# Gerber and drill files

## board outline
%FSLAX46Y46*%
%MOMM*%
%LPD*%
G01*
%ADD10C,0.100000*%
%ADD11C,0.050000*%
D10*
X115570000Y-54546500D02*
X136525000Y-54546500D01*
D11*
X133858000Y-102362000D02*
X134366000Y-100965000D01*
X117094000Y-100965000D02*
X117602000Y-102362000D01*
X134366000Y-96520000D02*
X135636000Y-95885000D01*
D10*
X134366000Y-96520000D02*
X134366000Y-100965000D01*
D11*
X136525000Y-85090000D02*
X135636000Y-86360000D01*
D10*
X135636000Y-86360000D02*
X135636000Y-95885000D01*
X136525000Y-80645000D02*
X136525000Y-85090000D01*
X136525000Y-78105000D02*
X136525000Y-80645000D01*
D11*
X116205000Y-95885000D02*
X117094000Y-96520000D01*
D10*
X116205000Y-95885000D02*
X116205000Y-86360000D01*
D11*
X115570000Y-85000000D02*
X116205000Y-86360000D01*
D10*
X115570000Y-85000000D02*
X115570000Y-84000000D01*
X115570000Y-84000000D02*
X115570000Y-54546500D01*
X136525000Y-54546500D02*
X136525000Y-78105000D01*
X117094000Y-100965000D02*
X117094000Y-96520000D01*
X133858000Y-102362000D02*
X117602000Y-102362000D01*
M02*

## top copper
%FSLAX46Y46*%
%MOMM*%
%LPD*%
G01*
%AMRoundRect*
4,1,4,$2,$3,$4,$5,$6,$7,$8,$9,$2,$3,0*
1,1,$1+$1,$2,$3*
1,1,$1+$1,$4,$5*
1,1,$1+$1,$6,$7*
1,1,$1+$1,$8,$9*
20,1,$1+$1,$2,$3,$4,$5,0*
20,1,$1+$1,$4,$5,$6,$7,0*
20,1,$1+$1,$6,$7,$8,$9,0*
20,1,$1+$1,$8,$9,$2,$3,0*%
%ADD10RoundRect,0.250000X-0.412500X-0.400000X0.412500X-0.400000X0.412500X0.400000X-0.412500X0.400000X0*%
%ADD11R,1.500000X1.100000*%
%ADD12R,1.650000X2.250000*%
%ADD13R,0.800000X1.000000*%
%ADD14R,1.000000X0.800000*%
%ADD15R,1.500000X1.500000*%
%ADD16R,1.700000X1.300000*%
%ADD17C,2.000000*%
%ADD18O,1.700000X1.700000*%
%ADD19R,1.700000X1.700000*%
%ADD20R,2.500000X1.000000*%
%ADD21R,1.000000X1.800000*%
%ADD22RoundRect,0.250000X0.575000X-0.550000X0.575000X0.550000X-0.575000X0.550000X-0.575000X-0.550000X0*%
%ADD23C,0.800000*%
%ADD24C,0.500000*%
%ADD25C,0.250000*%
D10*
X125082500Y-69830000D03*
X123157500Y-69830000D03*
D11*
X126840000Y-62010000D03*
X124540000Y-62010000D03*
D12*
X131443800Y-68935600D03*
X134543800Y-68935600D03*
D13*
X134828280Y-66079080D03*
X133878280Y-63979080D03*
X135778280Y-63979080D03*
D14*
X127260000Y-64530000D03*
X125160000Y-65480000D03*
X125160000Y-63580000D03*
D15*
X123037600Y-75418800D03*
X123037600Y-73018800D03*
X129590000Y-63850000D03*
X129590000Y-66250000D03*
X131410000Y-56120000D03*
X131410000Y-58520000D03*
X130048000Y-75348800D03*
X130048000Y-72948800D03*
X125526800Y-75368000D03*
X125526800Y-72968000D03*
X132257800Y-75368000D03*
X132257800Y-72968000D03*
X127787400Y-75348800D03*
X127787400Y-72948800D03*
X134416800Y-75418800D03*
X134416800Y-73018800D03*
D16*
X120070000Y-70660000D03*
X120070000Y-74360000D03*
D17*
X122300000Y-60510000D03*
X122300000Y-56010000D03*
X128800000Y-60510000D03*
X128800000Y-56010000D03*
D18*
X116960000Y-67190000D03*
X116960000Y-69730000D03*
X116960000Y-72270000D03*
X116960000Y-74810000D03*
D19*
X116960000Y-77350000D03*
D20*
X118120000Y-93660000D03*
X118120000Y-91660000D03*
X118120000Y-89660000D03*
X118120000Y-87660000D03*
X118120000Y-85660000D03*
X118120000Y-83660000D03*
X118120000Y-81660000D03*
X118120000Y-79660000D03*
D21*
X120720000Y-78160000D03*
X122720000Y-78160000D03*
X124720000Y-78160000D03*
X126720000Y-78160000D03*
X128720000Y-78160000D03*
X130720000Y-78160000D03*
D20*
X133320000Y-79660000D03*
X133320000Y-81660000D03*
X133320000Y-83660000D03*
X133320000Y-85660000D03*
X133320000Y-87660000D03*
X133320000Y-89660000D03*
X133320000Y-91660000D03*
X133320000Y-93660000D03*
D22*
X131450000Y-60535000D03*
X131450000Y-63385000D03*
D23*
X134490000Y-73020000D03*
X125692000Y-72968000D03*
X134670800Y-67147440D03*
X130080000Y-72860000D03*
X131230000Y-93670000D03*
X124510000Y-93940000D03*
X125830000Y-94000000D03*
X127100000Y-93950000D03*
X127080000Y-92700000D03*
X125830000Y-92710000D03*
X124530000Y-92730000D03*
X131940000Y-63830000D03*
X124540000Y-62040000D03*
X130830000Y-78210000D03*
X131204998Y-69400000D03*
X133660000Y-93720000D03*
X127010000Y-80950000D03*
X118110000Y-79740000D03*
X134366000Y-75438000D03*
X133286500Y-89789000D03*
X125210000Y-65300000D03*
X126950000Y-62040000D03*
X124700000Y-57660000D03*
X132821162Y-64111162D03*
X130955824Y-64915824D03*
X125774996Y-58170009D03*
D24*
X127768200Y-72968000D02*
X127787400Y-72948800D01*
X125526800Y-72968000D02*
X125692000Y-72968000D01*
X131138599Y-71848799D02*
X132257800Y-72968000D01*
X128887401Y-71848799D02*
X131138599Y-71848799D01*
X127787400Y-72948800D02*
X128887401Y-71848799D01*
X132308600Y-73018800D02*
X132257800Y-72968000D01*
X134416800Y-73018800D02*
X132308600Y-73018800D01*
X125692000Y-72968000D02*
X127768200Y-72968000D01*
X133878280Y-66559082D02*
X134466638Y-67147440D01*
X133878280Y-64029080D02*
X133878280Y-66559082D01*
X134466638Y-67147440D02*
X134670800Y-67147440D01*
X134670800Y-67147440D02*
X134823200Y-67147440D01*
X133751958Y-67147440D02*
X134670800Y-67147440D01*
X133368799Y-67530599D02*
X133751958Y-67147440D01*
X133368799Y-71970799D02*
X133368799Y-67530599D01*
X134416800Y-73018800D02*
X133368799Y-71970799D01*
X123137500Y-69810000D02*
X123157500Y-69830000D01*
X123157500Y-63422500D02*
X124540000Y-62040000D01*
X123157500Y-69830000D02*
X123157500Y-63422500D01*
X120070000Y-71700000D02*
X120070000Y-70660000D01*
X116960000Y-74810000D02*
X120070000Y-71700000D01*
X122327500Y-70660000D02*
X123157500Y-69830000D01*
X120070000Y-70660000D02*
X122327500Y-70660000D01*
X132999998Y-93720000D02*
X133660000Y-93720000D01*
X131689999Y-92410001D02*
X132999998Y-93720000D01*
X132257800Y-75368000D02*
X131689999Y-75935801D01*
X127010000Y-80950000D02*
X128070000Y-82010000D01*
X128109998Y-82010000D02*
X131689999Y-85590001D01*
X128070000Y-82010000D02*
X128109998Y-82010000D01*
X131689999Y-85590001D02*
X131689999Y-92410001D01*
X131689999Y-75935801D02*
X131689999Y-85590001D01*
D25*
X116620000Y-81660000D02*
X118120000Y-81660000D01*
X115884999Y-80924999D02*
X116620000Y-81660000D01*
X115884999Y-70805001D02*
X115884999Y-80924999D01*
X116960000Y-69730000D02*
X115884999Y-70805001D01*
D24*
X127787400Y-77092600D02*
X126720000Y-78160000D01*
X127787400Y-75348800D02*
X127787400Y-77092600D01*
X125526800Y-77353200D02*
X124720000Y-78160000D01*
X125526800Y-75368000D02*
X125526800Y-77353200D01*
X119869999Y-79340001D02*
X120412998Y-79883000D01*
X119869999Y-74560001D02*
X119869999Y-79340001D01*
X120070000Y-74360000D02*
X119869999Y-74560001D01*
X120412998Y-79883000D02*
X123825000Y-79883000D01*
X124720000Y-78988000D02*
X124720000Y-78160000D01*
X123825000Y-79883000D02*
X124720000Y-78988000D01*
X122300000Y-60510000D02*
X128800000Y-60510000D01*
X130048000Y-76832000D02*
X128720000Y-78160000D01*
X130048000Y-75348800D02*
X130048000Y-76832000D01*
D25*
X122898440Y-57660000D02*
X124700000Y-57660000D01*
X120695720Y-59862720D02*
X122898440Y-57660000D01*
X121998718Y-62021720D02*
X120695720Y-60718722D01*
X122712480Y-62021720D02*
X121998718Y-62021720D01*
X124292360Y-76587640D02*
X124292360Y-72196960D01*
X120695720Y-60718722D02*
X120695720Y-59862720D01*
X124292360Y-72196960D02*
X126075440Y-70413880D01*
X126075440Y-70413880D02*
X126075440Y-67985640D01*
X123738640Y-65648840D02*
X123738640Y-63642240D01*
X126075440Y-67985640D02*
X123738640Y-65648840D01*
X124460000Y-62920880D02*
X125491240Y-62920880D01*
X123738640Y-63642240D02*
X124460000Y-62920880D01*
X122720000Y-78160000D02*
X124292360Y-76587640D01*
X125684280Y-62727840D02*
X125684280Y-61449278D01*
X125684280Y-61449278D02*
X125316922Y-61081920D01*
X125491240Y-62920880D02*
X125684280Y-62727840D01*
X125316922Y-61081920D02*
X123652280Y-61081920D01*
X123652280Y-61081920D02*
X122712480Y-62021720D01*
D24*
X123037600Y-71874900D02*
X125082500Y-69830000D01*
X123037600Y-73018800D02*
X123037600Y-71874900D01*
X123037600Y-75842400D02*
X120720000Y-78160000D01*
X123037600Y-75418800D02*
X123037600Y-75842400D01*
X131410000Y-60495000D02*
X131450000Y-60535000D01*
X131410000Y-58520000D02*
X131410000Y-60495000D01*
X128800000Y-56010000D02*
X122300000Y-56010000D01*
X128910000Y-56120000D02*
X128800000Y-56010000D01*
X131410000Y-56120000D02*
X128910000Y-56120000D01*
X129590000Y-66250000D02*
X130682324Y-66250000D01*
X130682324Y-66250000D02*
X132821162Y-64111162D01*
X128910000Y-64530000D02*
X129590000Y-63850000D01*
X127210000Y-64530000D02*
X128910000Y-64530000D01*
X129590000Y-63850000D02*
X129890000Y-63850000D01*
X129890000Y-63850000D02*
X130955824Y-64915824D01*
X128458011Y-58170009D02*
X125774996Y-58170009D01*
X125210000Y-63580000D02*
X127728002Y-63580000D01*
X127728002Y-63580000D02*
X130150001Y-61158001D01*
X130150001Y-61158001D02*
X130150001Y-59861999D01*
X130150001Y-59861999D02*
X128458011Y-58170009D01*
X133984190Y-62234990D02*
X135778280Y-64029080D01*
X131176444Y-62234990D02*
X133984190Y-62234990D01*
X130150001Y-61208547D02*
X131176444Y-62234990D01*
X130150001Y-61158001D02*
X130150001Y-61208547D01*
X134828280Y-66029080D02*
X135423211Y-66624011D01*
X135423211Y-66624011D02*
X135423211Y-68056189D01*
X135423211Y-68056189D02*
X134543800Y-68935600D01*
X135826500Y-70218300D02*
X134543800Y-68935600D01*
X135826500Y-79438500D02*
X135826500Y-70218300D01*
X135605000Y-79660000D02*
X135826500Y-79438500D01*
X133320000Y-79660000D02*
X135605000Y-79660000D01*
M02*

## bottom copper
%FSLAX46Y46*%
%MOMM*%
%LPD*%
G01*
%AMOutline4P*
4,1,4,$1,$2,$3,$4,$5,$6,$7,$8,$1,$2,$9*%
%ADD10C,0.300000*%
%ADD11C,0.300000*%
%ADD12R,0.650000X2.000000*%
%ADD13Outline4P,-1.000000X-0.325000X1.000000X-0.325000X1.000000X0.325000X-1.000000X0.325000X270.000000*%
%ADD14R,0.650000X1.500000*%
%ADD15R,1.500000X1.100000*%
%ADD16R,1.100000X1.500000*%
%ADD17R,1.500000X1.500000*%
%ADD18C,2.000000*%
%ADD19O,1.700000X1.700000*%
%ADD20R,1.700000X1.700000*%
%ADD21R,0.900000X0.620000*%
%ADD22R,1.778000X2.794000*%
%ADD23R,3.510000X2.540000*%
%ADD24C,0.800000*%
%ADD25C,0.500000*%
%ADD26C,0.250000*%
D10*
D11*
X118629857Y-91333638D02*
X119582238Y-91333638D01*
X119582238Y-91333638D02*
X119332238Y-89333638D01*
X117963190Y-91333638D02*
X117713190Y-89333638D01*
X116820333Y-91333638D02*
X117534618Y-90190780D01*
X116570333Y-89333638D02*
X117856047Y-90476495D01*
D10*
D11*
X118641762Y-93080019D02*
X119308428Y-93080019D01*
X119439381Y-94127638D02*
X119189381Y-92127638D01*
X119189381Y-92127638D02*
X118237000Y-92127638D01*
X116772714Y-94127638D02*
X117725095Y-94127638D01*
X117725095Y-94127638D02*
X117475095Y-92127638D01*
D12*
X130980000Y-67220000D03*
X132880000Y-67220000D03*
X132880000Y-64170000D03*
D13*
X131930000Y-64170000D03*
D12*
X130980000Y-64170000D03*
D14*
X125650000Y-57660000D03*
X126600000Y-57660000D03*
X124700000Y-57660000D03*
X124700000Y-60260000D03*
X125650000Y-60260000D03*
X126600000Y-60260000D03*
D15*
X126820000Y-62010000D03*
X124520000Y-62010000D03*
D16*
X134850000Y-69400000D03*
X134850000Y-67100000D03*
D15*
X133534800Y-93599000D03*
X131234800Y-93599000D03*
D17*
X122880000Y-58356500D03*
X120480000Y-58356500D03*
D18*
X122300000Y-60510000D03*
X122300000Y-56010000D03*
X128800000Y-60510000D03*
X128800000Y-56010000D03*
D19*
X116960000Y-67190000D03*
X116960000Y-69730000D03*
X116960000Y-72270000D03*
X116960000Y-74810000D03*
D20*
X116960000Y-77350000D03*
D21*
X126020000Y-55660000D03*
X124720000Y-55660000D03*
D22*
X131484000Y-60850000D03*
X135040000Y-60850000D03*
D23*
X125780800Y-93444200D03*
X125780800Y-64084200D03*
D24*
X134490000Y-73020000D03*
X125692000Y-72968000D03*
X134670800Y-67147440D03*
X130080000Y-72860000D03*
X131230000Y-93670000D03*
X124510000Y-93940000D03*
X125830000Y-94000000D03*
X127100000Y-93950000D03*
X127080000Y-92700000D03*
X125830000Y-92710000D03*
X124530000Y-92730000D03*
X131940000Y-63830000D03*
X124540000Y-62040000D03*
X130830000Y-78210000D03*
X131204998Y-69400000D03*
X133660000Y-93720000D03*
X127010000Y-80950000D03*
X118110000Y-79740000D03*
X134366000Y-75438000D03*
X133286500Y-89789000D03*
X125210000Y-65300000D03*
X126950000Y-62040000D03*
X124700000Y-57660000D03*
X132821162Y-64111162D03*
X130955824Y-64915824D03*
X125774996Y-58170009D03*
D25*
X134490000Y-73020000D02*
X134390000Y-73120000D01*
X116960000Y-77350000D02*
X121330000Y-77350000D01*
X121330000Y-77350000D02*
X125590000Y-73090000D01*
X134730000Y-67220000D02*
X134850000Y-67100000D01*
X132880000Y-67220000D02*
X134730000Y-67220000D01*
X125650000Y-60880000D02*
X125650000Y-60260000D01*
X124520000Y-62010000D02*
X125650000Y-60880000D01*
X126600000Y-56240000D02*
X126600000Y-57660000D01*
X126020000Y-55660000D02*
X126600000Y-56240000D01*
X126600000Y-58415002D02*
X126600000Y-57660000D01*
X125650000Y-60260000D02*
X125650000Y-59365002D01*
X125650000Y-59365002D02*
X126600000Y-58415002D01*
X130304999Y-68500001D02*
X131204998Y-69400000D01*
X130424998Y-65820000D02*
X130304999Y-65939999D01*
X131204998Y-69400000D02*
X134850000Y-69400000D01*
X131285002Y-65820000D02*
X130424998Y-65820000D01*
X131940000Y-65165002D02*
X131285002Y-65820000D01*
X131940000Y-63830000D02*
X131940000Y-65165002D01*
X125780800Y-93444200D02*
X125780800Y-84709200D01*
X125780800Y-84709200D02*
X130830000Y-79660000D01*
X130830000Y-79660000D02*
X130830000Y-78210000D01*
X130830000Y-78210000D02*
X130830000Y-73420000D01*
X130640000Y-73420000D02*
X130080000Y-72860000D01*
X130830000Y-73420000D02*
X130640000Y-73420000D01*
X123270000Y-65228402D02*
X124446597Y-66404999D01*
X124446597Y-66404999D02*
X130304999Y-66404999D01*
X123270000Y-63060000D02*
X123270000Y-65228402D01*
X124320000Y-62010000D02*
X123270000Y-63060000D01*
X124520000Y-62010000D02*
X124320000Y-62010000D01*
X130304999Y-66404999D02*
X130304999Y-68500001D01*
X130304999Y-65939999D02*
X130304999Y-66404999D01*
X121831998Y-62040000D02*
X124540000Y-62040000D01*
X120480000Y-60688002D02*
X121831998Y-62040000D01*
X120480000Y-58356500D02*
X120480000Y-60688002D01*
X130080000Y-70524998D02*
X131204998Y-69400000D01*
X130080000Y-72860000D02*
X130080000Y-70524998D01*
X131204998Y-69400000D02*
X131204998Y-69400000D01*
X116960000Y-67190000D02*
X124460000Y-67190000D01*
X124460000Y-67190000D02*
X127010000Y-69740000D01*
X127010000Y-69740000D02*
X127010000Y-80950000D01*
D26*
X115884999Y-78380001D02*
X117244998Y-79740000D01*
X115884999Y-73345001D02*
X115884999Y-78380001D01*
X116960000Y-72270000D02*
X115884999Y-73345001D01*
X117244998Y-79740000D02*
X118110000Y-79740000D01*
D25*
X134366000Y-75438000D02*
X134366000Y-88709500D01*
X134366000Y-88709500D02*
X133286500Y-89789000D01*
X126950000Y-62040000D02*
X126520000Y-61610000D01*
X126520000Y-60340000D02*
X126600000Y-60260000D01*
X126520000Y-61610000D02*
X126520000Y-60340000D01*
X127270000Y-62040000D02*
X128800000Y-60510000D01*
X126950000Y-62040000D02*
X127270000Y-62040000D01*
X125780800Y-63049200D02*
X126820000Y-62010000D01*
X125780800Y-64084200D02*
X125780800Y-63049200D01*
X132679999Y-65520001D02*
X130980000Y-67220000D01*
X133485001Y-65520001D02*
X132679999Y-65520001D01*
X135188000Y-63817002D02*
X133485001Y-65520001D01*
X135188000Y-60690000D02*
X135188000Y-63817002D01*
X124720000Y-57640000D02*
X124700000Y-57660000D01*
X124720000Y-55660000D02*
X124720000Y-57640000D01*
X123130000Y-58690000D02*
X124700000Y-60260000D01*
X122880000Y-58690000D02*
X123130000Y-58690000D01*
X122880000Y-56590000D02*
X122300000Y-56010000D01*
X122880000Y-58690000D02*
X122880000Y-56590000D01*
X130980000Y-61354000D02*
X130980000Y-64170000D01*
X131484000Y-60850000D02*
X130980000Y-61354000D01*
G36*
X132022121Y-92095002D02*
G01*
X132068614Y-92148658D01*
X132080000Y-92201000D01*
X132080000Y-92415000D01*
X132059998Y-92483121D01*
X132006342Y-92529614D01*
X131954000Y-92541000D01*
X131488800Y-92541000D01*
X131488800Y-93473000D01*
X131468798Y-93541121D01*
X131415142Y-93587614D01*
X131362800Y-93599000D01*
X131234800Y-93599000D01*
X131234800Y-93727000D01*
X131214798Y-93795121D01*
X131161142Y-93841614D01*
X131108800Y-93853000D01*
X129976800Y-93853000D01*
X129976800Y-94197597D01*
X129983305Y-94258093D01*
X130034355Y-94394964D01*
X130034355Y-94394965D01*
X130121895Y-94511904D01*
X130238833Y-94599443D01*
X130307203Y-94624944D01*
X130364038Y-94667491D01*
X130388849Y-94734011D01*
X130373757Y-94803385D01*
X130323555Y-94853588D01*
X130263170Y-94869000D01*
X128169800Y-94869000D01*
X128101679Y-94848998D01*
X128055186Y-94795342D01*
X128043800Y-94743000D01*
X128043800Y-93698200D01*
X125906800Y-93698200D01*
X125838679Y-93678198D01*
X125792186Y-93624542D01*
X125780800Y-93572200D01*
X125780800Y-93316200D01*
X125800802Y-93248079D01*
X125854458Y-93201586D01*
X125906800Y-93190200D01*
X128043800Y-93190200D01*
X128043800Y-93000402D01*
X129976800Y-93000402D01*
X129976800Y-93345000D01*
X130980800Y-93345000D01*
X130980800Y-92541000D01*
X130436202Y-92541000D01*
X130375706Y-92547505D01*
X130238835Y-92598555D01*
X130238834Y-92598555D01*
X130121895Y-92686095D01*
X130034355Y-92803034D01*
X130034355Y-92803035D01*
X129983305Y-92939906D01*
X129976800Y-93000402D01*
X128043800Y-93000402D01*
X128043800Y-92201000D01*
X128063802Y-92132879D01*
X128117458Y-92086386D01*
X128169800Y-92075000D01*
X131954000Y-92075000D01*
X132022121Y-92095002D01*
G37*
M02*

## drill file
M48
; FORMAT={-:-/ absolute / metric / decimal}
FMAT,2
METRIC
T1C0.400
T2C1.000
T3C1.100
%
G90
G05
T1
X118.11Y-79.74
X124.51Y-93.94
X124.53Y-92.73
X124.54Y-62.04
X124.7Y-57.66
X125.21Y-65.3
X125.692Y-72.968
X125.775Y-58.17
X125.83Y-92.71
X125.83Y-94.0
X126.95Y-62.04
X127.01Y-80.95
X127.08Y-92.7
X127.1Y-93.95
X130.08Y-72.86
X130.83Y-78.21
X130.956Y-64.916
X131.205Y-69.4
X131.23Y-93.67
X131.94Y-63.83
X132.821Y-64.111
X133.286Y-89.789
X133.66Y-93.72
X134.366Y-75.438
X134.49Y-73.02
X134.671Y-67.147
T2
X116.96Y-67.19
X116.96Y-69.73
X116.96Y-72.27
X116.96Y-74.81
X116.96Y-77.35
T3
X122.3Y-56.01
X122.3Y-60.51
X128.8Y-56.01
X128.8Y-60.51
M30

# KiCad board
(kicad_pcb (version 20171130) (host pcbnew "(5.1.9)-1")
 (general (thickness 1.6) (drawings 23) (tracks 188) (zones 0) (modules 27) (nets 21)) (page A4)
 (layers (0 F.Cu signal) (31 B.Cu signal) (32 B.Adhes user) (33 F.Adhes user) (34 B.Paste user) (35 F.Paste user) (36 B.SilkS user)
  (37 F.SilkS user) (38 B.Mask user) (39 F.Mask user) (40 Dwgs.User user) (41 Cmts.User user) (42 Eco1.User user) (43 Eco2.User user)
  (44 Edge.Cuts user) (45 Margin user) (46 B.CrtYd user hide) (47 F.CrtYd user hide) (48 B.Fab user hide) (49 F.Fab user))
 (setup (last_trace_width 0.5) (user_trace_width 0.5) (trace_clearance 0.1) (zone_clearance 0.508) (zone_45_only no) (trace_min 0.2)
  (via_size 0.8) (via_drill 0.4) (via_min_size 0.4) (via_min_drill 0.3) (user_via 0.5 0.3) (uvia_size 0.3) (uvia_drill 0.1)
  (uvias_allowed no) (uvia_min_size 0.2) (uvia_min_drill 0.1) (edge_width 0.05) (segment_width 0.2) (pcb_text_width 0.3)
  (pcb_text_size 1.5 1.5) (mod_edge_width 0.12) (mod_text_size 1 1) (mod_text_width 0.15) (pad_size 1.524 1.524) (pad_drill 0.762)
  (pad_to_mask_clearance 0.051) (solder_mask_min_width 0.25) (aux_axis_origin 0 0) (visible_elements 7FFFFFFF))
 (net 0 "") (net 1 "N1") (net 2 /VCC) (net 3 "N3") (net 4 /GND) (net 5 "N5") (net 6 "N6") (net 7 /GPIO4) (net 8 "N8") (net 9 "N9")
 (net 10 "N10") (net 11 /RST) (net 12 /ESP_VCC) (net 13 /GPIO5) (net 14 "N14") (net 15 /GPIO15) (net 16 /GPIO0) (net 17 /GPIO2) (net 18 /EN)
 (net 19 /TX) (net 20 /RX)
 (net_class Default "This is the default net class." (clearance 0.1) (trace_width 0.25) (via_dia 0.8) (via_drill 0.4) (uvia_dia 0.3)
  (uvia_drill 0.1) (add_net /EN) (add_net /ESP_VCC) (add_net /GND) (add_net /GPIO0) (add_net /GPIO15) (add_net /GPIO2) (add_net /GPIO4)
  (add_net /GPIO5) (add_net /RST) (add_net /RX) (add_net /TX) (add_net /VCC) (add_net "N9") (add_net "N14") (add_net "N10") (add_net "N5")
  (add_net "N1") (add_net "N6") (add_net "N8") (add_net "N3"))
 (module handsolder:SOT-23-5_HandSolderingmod (layer B.Cu) (at 131.93 65.72 270)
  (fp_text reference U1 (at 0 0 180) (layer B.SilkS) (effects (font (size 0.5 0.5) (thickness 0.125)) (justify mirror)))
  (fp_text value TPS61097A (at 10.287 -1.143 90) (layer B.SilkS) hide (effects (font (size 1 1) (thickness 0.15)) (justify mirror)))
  (pad 5 smd rect (at 1.5 0.95 270) (size 2 0.65) (layers B.Cu B.Paste B.Mask) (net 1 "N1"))
  (pad 4 smd rect (at 1.5 -0.95 270) (size 2 0.65) (layers B.Cu B.Paste B.Mask) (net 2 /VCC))
  (pad 3 smd rect (at -1.55 -0.95 270) (size 2 0.65) (layers B.Cu B.Paste B.Mask) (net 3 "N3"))
  (pad 2 smd trapezoid (at -1.55 0 270) (size 2 0.65) (layers B.Cu B.Paste B.Mask) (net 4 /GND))
  (pad 1 smd rect (at -1.55 0.95 270) (size 2 0.65) (layers B.Cu B.Paste B.Mask) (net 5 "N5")))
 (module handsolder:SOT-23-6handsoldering (layer B.Cu) (at 125.65 58.96 90)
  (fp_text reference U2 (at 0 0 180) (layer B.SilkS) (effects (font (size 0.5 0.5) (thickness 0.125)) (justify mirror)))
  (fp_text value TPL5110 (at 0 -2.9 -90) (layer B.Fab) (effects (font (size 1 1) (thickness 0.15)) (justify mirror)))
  (pad 5 smd rect (at 1.3 0 90) (size 1.5 0.65) (layers B.Cu B.Paste B.Mask) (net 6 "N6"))
  (pad 6 smd rect (at 1.3 0.95 90) (size 1.5 0.65) (layers B.Cu B.Paste B.Mask) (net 4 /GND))
  (pad 4 smd rect (at 1.3 -0.95 90) (size 1.5 0.65) (layers B.Cu B.Paste B.Mask) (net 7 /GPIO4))
  (pad 3 smd rect (at -1.3 -0.95 90) (size 1.5 0.65) (layers B.Cu B.Paste B.Mask) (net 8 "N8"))
  (pad 2 smd rect (at -1.3 0 90) (size 1.5 0.65) (layers B.Cu B.Paste B.Mask) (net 4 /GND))
  (pad 1 smd rect (at -1.3 0.95 90) (size 1.5 0.65) (layers B.Cu B.Paste B.Mask) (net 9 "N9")))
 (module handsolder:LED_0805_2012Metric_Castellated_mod (layer F.Cu) (at 124.12 69.83)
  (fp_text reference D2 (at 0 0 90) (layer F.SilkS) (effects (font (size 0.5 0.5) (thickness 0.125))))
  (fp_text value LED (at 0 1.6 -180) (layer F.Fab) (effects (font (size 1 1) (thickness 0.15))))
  (pad 2 smd roundrect (at 0.9625 0) (size 1.325 1.3) (layers F.Cu F.Paste F.Mask) (roundrect_rratio 0.1923076923076923) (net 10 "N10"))
  (pad 1 smd roundrect (at -0.9625 0) (size 1.325 1.3) (layers F.Cu F.Paste F.Mask) (roundrect_rratio 0.1923076923076923) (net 4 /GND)))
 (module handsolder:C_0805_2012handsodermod (layer F.Cu) (at 125.69 62.01)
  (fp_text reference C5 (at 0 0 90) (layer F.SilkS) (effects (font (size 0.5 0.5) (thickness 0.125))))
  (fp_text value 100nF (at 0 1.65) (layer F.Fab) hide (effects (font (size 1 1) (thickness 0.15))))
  (pad 2 smd rect (at 1.15 0) (size 1.5 1.1) (layers F.Cu F.Paste F.Mask) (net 9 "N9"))
  (pad 1 smd rect (at -1.15 0) (size 1.5 1.1) (layers F.Cu F.Paste F.Mask) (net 4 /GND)))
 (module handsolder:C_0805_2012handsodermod (layer B.Cu) (at 125.67 62.01)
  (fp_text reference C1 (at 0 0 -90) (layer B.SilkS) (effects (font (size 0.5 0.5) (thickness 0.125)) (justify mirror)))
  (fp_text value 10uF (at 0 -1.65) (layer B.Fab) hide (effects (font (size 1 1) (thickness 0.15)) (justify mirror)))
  (pad 2 smd rect (at 1.15 0) (size 1.5 1.1) (layers B.Cu B.Paste B.Mask) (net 9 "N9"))
  (pad 1 smd rect (at -1.15 0) (size 1.5 1.1) (layers B.Cu B.Paste B.Mask) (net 4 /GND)))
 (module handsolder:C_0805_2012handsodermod (layer B.Cu) (at 134.85 68.25 270)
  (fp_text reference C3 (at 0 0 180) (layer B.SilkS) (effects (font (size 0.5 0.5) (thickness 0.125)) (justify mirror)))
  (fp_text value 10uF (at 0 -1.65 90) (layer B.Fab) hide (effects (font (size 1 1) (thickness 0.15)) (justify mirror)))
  (pad 2 smd rect (at 1.15 0 270) (size 1.5 1.1) (layers B.Cu B.Paste B.Mask) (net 4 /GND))
  (pad 1 smd rect (at -1.15 0 270) (size 1.5 1.1) (layers B.Cu B.Paste B.Mask) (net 2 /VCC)))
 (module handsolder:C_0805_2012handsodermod (layer B.Cu) (at 132.3848 93.599)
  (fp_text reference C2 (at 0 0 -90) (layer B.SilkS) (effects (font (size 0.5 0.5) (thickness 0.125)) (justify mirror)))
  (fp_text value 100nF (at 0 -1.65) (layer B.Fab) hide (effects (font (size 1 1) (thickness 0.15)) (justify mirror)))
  (pad 2 smd rect (at 1.15 0) (size 1.5 1.1) (layers B.Cu B.Paste B.Mask) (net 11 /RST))
  (pad 1 smd rect (at -1.15 0) (size 1.5 1.1) (layers B.Cu B.Paste B.Mask) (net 4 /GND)))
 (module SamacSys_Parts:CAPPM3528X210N (layer F.Cu) (at 132.9938 68.9356 180)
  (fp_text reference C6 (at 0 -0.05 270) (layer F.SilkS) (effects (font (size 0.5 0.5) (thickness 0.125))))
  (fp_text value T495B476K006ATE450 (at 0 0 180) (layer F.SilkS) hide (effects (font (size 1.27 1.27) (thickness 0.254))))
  (pad 2 smd rect (at 1.55 0 180) (size 1.65 2.25) (layers F.Cu F.Paste F.Mask) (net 4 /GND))
  (pad 1 smd rect (at -1.55 0 180) (size 1.65 2.25) (layers F.Cu F.Paste F.Mask) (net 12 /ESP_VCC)))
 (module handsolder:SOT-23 (layer F.Cu) (at 134.82828 65.02908 270)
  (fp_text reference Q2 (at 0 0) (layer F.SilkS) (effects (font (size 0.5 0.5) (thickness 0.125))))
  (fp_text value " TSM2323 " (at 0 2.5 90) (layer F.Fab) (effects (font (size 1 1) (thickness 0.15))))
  (pad 3 smd rect (at 1.05 0 270) (size 1 0.8) (layers F.Cu F.Paste F.Mask) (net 12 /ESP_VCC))
  (pad 2 smd rect (at -1.05 0.95 270) (size 1 0.8) (layers F.Cu F.Paste F.Mask) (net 2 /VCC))
  (pad 1 smd rect (at -1.05 -0.95 270) (size 1 0.8) (layers F.Cu F.Paste F.Mask) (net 6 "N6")))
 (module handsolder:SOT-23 (layer F.Cu) (at 126.21 64.53)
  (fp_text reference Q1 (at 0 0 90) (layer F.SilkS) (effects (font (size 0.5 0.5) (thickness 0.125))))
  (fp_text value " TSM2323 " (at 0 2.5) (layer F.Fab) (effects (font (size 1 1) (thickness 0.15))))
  (pad 3 smd rect (at 1.05 0) (size 1 0.8) (layers F.Cu F.Paste F.Mask) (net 5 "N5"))
  (pad 2 smd rect (at -1.05 0.95) (size 1 0.8) (layers F.Cu F.Paste F.Mask) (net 9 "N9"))
  (pad 1 smd rect (at -1.05 -0.95) (size 1 0.8) (layers F.Cu F.Paste F.Mask) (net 6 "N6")))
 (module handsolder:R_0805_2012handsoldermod (layer F.Cu) (at 123.0376 74.2188 270)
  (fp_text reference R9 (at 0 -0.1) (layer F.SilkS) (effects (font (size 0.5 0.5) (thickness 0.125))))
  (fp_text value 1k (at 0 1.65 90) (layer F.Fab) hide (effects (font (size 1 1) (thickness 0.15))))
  (pad 2 smd rect (at 1.2 0 270) (size 1.5 1.5) (layers F.Cu F.Paste F.Mask) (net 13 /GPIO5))
  (pad 1 smd rect (at -1.2 0 270) (size 1.5 1.5) (layers F.Cu F.Paste F.Mask) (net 10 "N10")))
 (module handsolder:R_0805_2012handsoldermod (layer B.Cu) (at 121.68 58.3565)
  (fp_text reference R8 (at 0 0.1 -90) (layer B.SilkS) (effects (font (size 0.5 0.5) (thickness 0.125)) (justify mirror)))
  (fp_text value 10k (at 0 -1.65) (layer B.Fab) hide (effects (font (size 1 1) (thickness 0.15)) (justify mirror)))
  (pad 2 smd rect (at 1.2 0) (size 1.5 1.5) (layers B.Cu B.Paste B.Mask) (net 8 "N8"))
  (pad 1 smd rect (at -1.2 0) (size 1.5 1.5) (layers B.Cu B.Paste B.Mask) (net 4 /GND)))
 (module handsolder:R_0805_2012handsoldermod (layer F.Cu) (at 129.59 65.05 90)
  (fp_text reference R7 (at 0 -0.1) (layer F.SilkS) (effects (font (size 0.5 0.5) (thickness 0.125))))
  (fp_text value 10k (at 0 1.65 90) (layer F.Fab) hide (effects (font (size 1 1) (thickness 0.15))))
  (pad 2 smd rect (at 1.2 0 90) (size 1.5 1.5) (layers F.Cu F.Paste F.Mask) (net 5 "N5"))
  (pad 1 smd rect (at -1.2 0 90) (size 1.5 1.5) (layers F.Cu F.Paste F.Mask) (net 3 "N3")))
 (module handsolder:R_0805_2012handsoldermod (layer F.Cu) (at 131.41 57.32 90)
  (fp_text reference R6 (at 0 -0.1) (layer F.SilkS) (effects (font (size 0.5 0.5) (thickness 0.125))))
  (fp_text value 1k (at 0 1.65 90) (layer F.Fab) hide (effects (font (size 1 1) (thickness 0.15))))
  (pad 2 smd rect (at 1.2 0 90) (size 1.5 1.5) (layers F.Cu F.Paste F.Mask) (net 8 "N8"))
  (pad 1 smd rect (at -1.2 0 90) (size 1.5 1.5) (layers F.Cu F.Paste F.Mask) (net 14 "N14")))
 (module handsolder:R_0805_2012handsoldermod (layer F.Cu) (at 130.048 74.1488 270)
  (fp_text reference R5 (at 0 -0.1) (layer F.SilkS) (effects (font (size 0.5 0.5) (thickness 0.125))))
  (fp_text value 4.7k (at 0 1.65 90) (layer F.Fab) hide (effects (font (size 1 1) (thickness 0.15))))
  (pad 2 smd rect (at 1.2 0 270) (size 1.5 1.5) (layers F.Cu F.Paste F.Mask) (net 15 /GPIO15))
  (pad 1 smd rect (at -1.2 0 270) (size 1.5 1.5) (layers F.Cu F.Paste F.Mask) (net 4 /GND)))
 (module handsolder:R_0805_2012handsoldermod (layer F.Cu) (at 125.5268 74.168 270)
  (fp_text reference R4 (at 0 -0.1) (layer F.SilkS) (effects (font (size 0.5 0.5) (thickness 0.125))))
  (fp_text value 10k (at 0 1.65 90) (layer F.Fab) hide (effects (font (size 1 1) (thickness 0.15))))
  (pad 2 smd rect (at 1.2 0 270) (size 1.5 1.5) (layers F.Cu F.Paste F.Mask) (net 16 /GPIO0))
  (pad 1 smd rect (at -1.2 0 270) (size 1.5 1.5) (layers F.Cu F.Paste F.Mask) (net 2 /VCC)))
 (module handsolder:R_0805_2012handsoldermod (layer F.Cu) (at 132.2578 74.168 270)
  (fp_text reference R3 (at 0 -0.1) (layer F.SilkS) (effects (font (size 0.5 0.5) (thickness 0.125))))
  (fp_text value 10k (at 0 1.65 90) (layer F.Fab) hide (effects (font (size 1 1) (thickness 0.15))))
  (pad 2 smd rect (at 1.2 0 270) (size 1.5 1.5) (layers F.Cu F.Paste F.Mask) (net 11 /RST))
  (pad 1 smd rect (at -1.2 0 270) (size 1.5 1.5) (layers F.Cu F.Paste F.Mask) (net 2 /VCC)))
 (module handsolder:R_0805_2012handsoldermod (layer F.Cu) (at 127.7874 74.1488 270)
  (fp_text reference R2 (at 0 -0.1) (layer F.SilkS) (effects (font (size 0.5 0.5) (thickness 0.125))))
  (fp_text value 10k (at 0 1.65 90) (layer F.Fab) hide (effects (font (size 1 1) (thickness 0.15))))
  (pad 2 smd rect (at 1.2 0 270) (size 1.5 1.5) (layers F.Cu F.Paste F.Mask) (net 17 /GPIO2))
  (pad 1 smd rect (at -1.2 0 270) (size 1.5 1.5) (layers F.Cu F.Paste F.Mask) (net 2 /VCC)))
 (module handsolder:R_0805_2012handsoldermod (layer F.Cu) (at 134.4168 74.2188 270)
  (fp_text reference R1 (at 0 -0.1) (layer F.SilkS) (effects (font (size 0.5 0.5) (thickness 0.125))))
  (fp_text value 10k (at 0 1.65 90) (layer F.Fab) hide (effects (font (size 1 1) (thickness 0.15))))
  (pad 2 smd rect (at 1.2 0 270) (size 1.5 1.5) (layers F.Cu F.Paste F.Mask) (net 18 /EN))
  (pad 1 smd rect (at -1.2 0 270) (size 1.5 1.5) (layers F.Cu F.Paste F.Mask) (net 2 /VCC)))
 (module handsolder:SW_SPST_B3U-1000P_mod (layer F.Cu) (at 120.07 72.51 90)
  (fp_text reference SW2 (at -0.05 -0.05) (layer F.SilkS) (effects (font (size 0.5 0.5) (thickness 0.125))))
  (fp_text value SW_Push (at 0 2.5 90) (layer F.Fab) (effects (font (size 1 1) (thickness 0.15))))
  (pad 2 smd rect (at 1.85 0 90) (size 1.3 1.7) (layers F.Cu F.Paste F.Mask) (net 4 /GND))
  (pad 1 smd rect (at -1.85 0 90) (size 1.3 1.7) (layers F.Cu F.Paste F.Mask) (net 16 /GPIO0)))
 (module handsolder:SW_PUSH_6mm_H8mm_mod (layer F.Cu) (at 128.8 60.51 180)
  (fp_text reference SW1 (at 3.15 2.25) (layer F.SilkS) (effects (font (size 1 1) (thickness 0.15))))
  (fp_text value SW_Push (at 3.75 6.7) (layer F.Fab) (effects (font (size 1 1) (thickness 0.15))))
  (pad 1 thru_hole circle (at 6.5 0 270) (size 2 2) (drill 1.1) (layers *.Cu *.Mask) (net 9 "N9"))
  (pad 2 thru_hole circle (at 6.5 4.5 270) (size 2 2) (drill 1.1) (layers *.Cu *.Mask) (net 8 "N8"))
  (pad 1 thru_hole circle (at 0 0 270) (size 2 2) (drill 1.1) (layers *.Cu *.Mask) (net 9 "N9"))
  (pad 2 thru_hole circle (at 0 4.5 270) (size 2 2) (drill 1.1) (layers *.Cu *.Mask) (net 8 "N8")))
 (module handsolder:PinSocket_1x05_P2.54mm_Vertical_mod (layer F.Cu) (at 116.96 77.35 180)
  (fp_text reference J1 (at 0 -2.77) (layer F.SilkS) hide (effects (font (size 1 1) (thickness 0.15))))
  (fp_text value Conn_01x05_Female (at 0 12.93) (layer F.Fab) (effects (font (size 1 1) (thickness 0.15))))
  (pad 5 thru_hole oval (at 0 10.16 180) (size 1.7 1.7) (drill 1) (layers *.Cu *.Mask) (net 11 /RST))
  (pad 4 thru_hole oval (at 0 7.62 180) (size 1.7 1.7) (drill 1) (layers *.Cu *.Mask) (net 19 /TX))
  (pad 3 thru_hole oval (at 0 5.08 180) (size 1.7 1.7) (drill 1) (layers *.Cu *.Mask) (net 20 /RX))
  (pad 2 thru_hole oval (at 0 2.54 180) (size 1.7 1.7) (drill 1) (layers *.Cu *.Mask) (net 4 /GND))
  (pad 1 thru_hole rect (at 0 0 180) (size 1.7 1.7) (drill 1) (layers *.Cu *.Mask) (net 2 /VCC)))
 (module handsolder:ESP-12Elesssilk (layer F.Cu) (at 125.72 90.16 180)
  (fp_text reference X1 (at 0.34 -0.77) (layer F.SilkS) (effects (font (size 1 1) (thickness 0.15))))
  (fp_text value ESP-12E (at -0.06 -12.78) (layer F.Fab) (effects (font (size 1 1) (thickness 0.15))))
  (pad 22 smd rect (at 7.6 -3.5 180) (size 2.5 1) (layers F.Cu F.Paste F.Mask))
  (pad 21 smd rect (at 7.6 -1.5 180) (size 2.5 1) (layers F.Cu F.Paste F.Mask))
  (pad 20 smd rect (at 7.6 0.5 180) (size 2.5 1) (layers F.Cu F.Paste F.Mask))
  (pad 19 smd rect (at 7.6 2.5 180) (size 2.5 1) (layers F.Cu F.Paste F.Mask))
  (pad 18 smd rect (at 7.6 4.5 180) (size 2.5 1) (layers F.Cu F.Paste F.Mask))
  (pad 17 smd rect (at 7.6 6.5 180) (size 2.5 1) (layers F.Cu F.Paste F.Mask))
  (pad 16 smd rect (at 7.6 8.5 180) (size 2.5 1) (layers F.Cu F.Paste F.Mask) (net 19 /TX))
  (pad 15 smd rect (at 7.6 10.5 180) (size 2.5 1) (layers F.Cu F.Paste F.Mask) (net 20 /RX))
  (pad 14 smd rect (at 5 12 180) (size 1 1.8) (layers F.Cu F.Paste F.Mask) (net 13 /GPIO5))
  (pad 13 smd rect (at 3 12 180) (size 1 1.8) (layers F.Cu F.Paste F.Mask) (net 7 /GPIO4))
  (pad 12 smd rect (at 1 12 180) (size 1 1.8) (layers F.Cu F.Paste F.Mask) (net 16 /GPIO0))
  (pad 11 smd rect (at -1 12 180) (size 1 1.8) (layers F.Cu F.Paste F.Mask) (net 17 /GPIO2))
  (pad 10 smd rect (at -3 12 180) (size 1 1.8) (layers F.Cu F.Paste F.Mask) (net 15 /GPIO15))
  (pad 9 smd rect (at -5 12 180) (size 1 1.8) (layers F.Cu F.Paste F.Mask) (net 4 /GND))
  (pad 8 smd rect (at -7.6 10.5 180) (size 2.5 1) (layers F.Cu F.Paste F.Mask) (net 12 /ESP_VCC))
  (pad 7 smd rect (at -7.6 8.5 180) (size 2.5 1) (layers F.Cu F.Paste F.Mask))
  (pad 6 smd rect (at -7.6 6.5 180) (size 2.5 1) (layers F.Cu F.Paste F.Mask))
  (pad 5 smd rect (at -7.6 4.5 180) (size 2.5 1) (layers F.Cu F.Paste F.Mask))
  (pad 4 smd rect (at -7.6 2.5 180) (size 2.5 1) (layers F.Cu F.Paste F.Mask))
  (pad 3 smd rect (at -7.6 0.5 180) (size 2.5 1) (layers F.Cu F.Paste F.Mask) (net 18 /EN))
  (pad 2 smd rect (at -7.6 -1.5 180) (size 2.5 1) (layers F.Cu F.Paste F.Mask))
  (pad 1 smd rect (at -7.6 -3.5 180) (size 2.5 1) (layers F.Cu F.Paste F.Mask) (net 11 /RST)))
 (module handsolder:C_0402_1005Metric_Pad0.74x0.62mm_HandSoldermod (layer B.Cu) (at 125.37 55.66)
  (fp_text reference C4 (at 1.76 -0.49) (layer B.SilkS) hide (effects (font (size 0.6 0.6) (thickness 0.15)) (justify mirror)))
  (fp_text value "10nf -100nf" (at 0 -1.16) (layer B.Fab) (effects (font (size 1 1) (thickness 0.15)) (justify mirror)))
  (pad 2 smd rect (at 0.65 0) (size 0.9 0.62) (layers B.Cu B.Paste B.Mask) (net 4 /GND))
  (pad 1 smd rect (at -0.65 0) (size 0.9 0.62) (layers B.Cu B.Paste B.Mask) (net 7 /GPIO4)))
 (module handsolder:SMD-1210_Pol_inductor (layer B.Cu) (at 133.262 60.85)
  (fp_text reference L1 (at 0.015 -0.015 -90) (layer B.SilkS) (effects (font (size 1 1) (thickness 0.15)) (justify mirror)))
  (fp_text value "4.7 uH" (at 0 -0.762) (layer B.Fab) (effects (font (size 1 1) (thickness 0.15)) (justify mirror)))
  (pad 1 smd rect (at -1.778 0) (size 1.778 2.794) (layers B.Cu B.Paste B.Mask) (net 5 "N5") (zone_connect 2))
  (pad 2 smd rect (at 1.778 0) (size 1.778 2.794) (layers B.Cu B.Paste B.Mask) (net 1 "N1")))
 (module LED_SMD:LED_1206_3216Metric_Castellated (layer F.Cu) (at 131.45 61.96 90)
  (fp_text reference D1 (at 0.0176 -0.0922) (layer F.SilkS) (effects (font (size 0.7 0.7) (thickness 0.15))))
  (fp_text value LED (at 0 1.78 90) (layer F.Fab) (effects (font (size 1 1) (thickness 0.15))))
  (pad 2 smd roundrect (at 1.425 0 90) (size 1.6 1.65) (layers F.Cu F.Paste F.Mask) (roundrect_rratio 0.15625) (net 14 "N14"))
  (pad 1 smd roundrect (at -1.425 0 90) (size 1.6 1.65) (layers F.Cu F.Paste F.Mask) (roundrect_rratio 0.15625) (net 4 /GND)))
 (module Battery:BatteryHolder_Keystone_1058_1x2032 (layer B.Cu) (at 125.7808 78.7642 270)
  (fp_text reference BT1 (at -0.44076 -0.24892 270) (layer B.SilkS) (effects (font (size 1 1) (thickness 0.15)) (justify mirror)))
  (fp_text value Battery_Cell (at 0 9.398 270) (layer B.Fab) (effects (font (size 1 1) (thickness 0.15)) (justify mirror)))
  (pad 2 smd rect (at 14.68 0 270) (size 2.54 3.51) (layers B.Cu B.Paste B.Mask) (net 4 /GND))
  (pad 1 smd rect (at -14.68 0 270) (size 2.54 3.51) (layers B.Cu B.Paste B.Mask) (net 9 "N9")))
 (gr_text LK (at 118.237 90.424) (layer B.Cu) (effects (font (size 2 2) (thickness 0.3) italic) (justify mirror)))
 (gr_line (start 115.57 54.5465) (end 136.525 54.5465) (layer Edge.Cuts) (width 0.1))
 (gr_line (start 133.858 102.362) (end 134.366 100.965) (layer Edge.Cuts) (width 0.05))
 (gr_line (start 117.094 100.965) (end 117.602 102.362) (layer Edge.Cuts) (width 0.05))
 (gr_line (start 134.366 96.52) (end 135.636 95.885) (layer Edge.Cuts) (width 0.05))
 (gr_line (start 134.366 96.52) (end 134.366 100.965) (layer Edge.Cuts) (width 0.1))
 (gr_line (start 136.525 85.09) (end 135.636 86.36) (layer Edge.Cuts) (width 0.05))
 (gr_line (start 135.636 86.36) (end 135.636 95.885) (layer Edge.Cuts) (width 0.1))
 (gr_line (start 136.525 80.645) (end 136.525 85.09) (layer Edge.Cuts) (width 0.1))
 (gr_line (start 136.525 78.105) (end 136.525 80.645) (layer Edge.Cuts) (width 0.1))
 (gr_line (start 116.205 95.885) (end 117.094 96.52) (layer Edge.Cuts) (width 0.05))
 (gr_line (start 116.205 95.885) (end 116.205 86.36) (layer Edge.Cuts) (width 0.1))
 (gr_line (start 115.57 85) (end 116.205 86.36) (layer Edge.Cuts) (width 0.05))
 (gr_line (start 115.57 85) (end 115.57 84) (layer Edge.Cuts) (width 0.1))
 (gr_line (start 115.57 84) (end 115.57 54.5465) (layer Edge.Cuts) (width 0.1))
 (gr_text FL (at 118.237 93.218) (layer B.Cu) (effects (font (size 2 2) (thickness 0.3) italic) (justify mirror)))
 (gr_line (start 136.525 54.5465) (end 136.525 78.105) (layer Edge.Cuts) (width 0.1))
 (gr_line (start 117.094 100.965) (end 117.094 96.52) (layer Edge.Cuts) (width 0.1))
 (gr_line (start 133.858 102.362) (end 117.602 102.362) (layer Edge.Cuts) (width 0.1))
 (segment (start 127.7682 72.968) (end 127.7874 72.9488) (width 0.5) (layer F.Cu) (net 2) (status 30))
 (segment (start 125.5268 72.968) (end 125.692 72.968) (width 0.5) (layer F.Cu) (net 2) (status 30))
 (segment (start 131.138599 71.848799) (end 132.2578 72.968) (width 0.5) (layer F.Cu) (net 2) (status 20))
 (segment (start 128.887401 71.848799) (end 131.138599 71.848799) (width 0.5) (layer F.Cu) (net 2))
 (segment (start 127.7874 72.9488) (end 128.887401 71.848799) (width 0.5) (layer F.Cu) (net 2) (status 10))
 (segment (start 132.3086 73.0188) (end 132.2578 72.968) (width 0.5) (layer F.Cu) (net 2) (status 30))
 (segment (start 134.4168 73.0188) (end 132.3086 73.0188) (width 0.5) (layer F.Cu) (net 2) (status 30))
 (segment (start 134.49 73.02) (end 134.39 73.12) (width 0.5) (layer B.Cu) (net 2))
 (via (at 134.49 73.02) (size 0.8) (drill 0.4) (layers F.Cu B.Cu) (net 2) (status 30))
 (segment (start 116.96 77.35) (end 121.33 77.35) (width 0.5) (layer B.Cu) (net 2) (status 10))
 (segment (start 121.33 77.35) (end 125.59 73.09) (width 0.5) (layer B.Cu) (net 2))
 (segment (start 125.692 72.968) (end 127.7682 72.968) (width 0.5) (layer F.Cu) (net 2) (status 30))
 (via (at 125.692 72.968) (size 0.8) (drill 0.4) (layers F.Cu B.Cu) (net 2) (status 30))
 (segment (start 134.73 67.22) (end 134.85 67.1) (width 0.5) (layer B.Cu) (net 2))
 (segment (start 132.88 67.22) (end 134.73 67.22) (width 0.5) (layer B.Cu) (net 2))
 (segment (start 133.87828 66.559082) (end 134.466638 67.14744) (width 0.5) (layer F.Cu) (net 2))
 (segment (start 133.87828 64.02908) (end 133.87828 66.559082) (width 0.5) (layer F.Cu) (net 2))
 (segment (start 134.466638 67.14744) (end 134.6708 67.14744) (width 0.5) (layer F.Cu) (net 2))
 (segment (start 134.6708 67.14744) (end 134.8232 67.14744) (width 0.5) (layer F.Cu) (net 2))
 (via (at 134.6708 67.14744) (size 0.8) (drill 0.4) (layers F.Cu B.Cu) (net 2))
 (segment (start 133.751958 67.14744) (end 134.6708 67.14744) (width 0.5) (layer F.Cu) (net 2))
 (segment (start 133.368799 67.530599) (end 133.751958 67.14744) (width 0.5) (layer F.Cu) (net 2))
 (segment (start 133.368799 71.970799) (end 133.368799 67.530599) (width 0.5) (layer F.Cu) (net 2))
 (segment (start 134.4168 73.0188) (end 133.368799 71.970799) (width 0.5) (layer F.Cu) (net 2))
 (via (at 130.08 72.86) (size 0.8) (drill 0.4) (layers F.Cu B.Cu) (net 4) (status 30))
 (via (at 131.23 93.67) (size 0.8) (drill 0.4) (layers F.Cu B.Cu) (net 4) (status 30))
 (via (at 124.51 93.94) (size 0.8) (drill 0.4) (layers F.Cu B.Cu) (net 4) (status 30))
 (via (at 125.83 94) (size 0.8) (drill 0.4) (layers F.Cu B.Cu) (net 4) (status 30))
 (via (at 127.1 93.95) (size 0.8) (drill 0.4) (layers F.Cu B.Cu) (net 4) (status 30))
 (via (at 127.08 92.7) (size 0.8) (drill 0.4) (layers F.Cu B.Cu) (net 4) (status 30))
 (via (at 125.83 92.71) (size 0.8) (drill 0.4) (layers F.Cu B.Cu) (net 4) (status 30))
 (via (at 124.53 92.73) (size 0.8) (drill 0.4) (layers F.Cu B.Cu) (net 4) (status 30))
 (via (at 131.94 63.83) (size 0.8) (drill 0.4) (layers F.Cu B.Cu) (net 4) (status 30))
 (via (at 124.54 62.04) (size 0.8) (drill 0.4) (layers F.Cu B.Cu) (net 4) (status 30))
 (segment (start 125.65 60.88) (end 125.65 60.26) (width 0.5) (layer B.Cu) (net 4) (status 20))
 (segment (start 124.52 62.01) (end 125.65 60.88) (width 0.5) (layer B.Cu) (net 4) (status 10))
 (segment (start 126.6 56.24) (end 126.6 57.66) (width 0.5) (layer B.Cu) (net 4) (status 20))
 (segment (start 126.02 55.66) (end 126.6 56.24) (width 0.5) (layer B.Cu) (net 4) (status 10))
 (segment (start 126.6 58.415002) (end 126.6 57.66) (width 0.5) (layer B.Cu) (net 4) (status 20))
 (segment (start 125.65 60.26) (end 125.65 59.365002) (width 0.5) (layer B.Cu) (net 4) (status 10))
 (segment (start 125.65 59.365002) (end 126.6 58.415002) (width 0.5) (layer B.Cu) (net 4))
 (segment (start 130.304999 68.500001) (end 131.204998 69.4) (width 0.5) (layer B.Cu) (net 4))
 (segment (start 130.424998 65.82) (end 130.304999 65.939999) (width 0.5) (layer B.Cu) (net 4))
 (segment (start 131.204998 69.4) (end 134.85 69.4) (width 0.5) (layer B.Cu) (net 4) (status 20))
 (segment (start 131.285002 65.82) (end 130.424998 65.82) (width 0.5) (layer B.Cu) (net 4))
 (segment (start 131.94 65.165002) (end 131.285002 65.82) (width 0.5) (layer B.Cu) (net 4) (status 10))
 (segment (start 131.94 63.83) (end 131.94 65.165002) (width 0.5) (layer B.Cu) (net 4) (status 30))
 (segment (start 125.7808 93.4442) (end 125.7808 84.7092) (width 0.5) (layer B.Cu) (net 4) (status 10))
 (segment (start 125.7808 84.7092) (end 130.83 79.66) (width 0.5) (layer B.Cu) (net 4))
 (segment (start 130.83 79.66) (end 130.83 78.21) (width 0.5) (layer B.Cu) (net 4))
 (via (at 130.83 78.21) (size 0.8) (drill 0.4) (layers F.Cu B.Cu) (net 4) (status 30))
 (segment (start 130.83 78.21) (end 130.83 73.42) (width 0.5) (layer B.Cu) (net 4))
 (segment (start 130.64 73.42) (end 130.08 72.86) (width 0.5) (layer B.Cu) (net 4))
 (segment (start 130.83 73.42) (end 130.64 73.42) (width 0.5) (layer B.Cu) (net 4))
 (segment (start 123.1375 69.81) (end 123.1575 69.83) (width 0.5) (layer F.Cu) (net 4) (status 30))
 (segment (start 123.1575 63.4225) (end 124.54 62.04) (width 0.5) (layer F.Cu) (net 4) (status 20))
 (segment (start 123.1575 69.83) (end 123.1575 63.4225) (width 0.5) (layer F.Cu) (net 4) (status 10))
 (segment (start 123.27 65.228402) (end 124.446597 66.404999) (width 0.5) (layer B.Cu) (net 4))
 (segment (start 124.446597 66.404999) (end 130.304999 66.404999) (width 0.5) (layer B.Cu) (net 4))
 (segment (start 123.27 63.06) (end 123.27 65.228402) (width 0.5) (layer B.Cu) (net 4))
 (segment (start 124.32 62.01) (end 123.27 63.06) (width 0.5) (layer B.Cu) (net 4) (status 10))
 (segment (start 124.52 62.01) (end 124.32 62.01) (width 0.5) (layer B.Cu) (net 4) (status 30))
 (segment (start 130.304999 66.404999) (end 130.304999 68.500001) (width 0.5) (layer B.Cu) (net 4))
 (segment (start 130.304999 65.939999) (end 130.304999 66.404999) (width 0.5) (layer B.Cu) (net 4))
 (segment (start 120.07 71.7) (end 120.07 70.66) (width 0.5) (layer F.Cu) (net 4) (status 20))
 (segment (start 116.96 74.81) (end 120.07 71.7) (width 0.5) (layer F.Cu) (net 4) (status 10))
 (segment (start 122.3275 70.66) (end 123.1575 69.83) (width 0.5) (layer F.Cu) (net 4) (status 20))
 (segment (start 120.07 70.66) (end 122.3275 70.66) (width 0.5) (layer F.Cu) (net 4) (status 10))
 (segment (start 121.831998 62.04) (end 124.54 62.04) (width 0.5) (layer B.Cu) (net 4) (status 20))
 (segment (start 120.48 60.688002) (end 121.831998 62.04) (width 0.5) (layer B.Cu) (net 4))
 (segment (start 120.48 58.3565) (end 120.48 60.688002) (width 0.5) (layer B.Cu) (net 4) (status 10))
 (segment (start 130.08 70.524998) (end 131.204998 69.4) (width 0.5) (layer B.Cu) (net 4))
 (segment (start 130.08 72.86) (end 130.08 70.524998) (width 0.5) (layer B.Cu) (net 4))
 (segment (start 131.204998 69.4) (end 131.204998 69.4) (width 0.5) (layer B.Cu) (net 4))
 (via (at 131.204998 69.4) (size 0.8) (drill 0.4) (layers F.Cu B.Cu) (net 4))
 (via (at 133.66 93.72) (size 0.8) (drill 0.4) (layers F.Cu B.Cu) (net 11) (status 30))
 (segment (start 132.999998 93.72) (end 133.66 93.72) (width 0.5) (layer F.Cu) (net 11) (status 30))
 (segment (start 131.689999 92.410001) (end 132.999998 93.72) (width 0.5) (layer F.Cu) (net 11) (status 20))
 (segment (start 132.2578 75.368) (end 131.689999 75.935801) (width 0.5) (layer F.Cu) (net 11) (status 30))
 (segment (start 116.96 67.19) (end 124.46 67.19) (width 0.5) (layer B.Cu) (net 11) (status 10))
 (segment (start 124.46 67.19) (end 127.01 69.74) (width 0.5) (layer B.Cu) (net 11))
 (segment (start 127.01 69.74) (end 127.01 80.95) (width 0.5) (layer B.Cu) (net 11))
 (via (at 127.01 80.95) (size 0.8) (drill 0.4) (layers F.Cu B.Cu) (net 11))
 (segment (start 127.01 80.95) (end 128.07 82.01) (width 0.5) (layer F.Cu) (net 11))
 (segment (start 128.109998 82.01) (end 131.689999 85.590001) (width 0.5) (layer F.Cu) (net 11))
 (segment (start 128.07 82.01) (end 128.109998 82.01) (width 0.5) (layer F.Cu) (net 11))
 (segment (start 131.689999 85.590001) (end 131.689999 92.410001) (width 0.5) (layer F.Cu) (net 11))
 (segment (start 131.689999 75.935801) (end 131.689999 85.590001) (width 0.5) (layer F.Cu) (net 11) (status 10))
 (segment (start 115.884999 78.380001) (end 117.244998 79.74) (width 0.25) (layer B.Cu) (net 20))
 (segment (start 115.884999 73.345001) (end 115.884999 78.380001) (width 0.25) (layer B.Cu) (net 20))
 (segment (start 116.96 72.27) (end 115.884999 73.345001) (width 0.25) (layer B.Cu) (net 20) (status 10))
 (segment (start 117.244998 79.74) (end 118.11 79.74) (width 0.25) (layer B.Cu) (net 20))
 (via (at 118.11 79.74) (size 0.8) (drill 0.4) (layers F.Cu B.Cu) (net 20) (status 30))
 (segment (start 116.62 81.66) (end 118.12 81.66) (width 0.25) (layer F.Cu) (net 19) (status 20))
 (segment (start 115.884999 80.924999) (end 116.62 81.66) (width 0.25) (layer F.Cu) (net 19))
 (segment (start 115.884999 70.805001) (end 115.884999 80.924999) (width 0.25) (layer F.Cu) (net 19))
 (segment (start 116.96 69.73) (end 115.884999 70.805001) (width 0.25) (layer F.Cu) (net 19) (status 10))
 (via (at 134.366 75.438) (size 0.8) (drill 0.4) (layers F.Cu B.Cu) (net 18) (status 30))
 (segment (start 134.366 75.438) (end 134.366 88.7095) (width 0.5) (layer B.Cu) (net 18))
 (segment (start 134.366 88.7095) (end 133.2865 89.789) (width 0.5) (layer B.Cu) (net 18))
 (via (at 133.2865 89.789) (size 0.8) (drill 0.4) (layers F.Cu B.Cu) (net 18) (status 30))
 (segment (start 127.7874 77.0926) (end 126.72 78.16) (width 0.5) (layer F.Cu) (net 17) (status 20))
 (segment (start 127.7874 75.3488) (end 127.7874 77.0926) (width 0.5) (layer F.Cu) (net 17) (status 10))
 (segment (start 125.5268 77.3532) (end 124.72 78.16) (width 0.5) (layer F.Cu) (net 16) (status 20))
 (segment (start 125.5268 75.368) (end 125.5268 77.3532) (width 0.5) (layer F.Cu) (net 16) (status 10))
 (segment (start 119.869999 79.340001) (end 120.412998 79.883) (width 0.5) (layer F.Cu) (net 16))
 (segment (start 119.869999 74.560001) (end 119.869999 79.340001) (width 0.5) (layer F.Cu) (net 16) (status 10))
 (segment (start 120.07 74.36) (end 119.869999 74.560001) (width 0.5) (layer F.Cu) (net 16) (status 30))
 (segment (start 120.412998 79.883) (end 123.825 79.883) (width 0.5) (layer F.Cu) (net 16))
 (segment (start 124.72 78.988) (end 124.72 78.16) (width 0.5) (layer F.Cu) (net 16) (status 30))
 (segment (start 123.825 79.883) (end 124.72 78.988) (width 0.5) (layer F.Cu) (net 16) (status 20))
 (via (at 125.21 65.3) (size 0.8) (drill 0.4) (layers F.Cu B.Cu) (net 9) (status 30))
 (via (at 126.95 62.04) (size 0.8) (drill 0.4) (layers F.Cu B.Cu) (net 9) (status 30))
 (segment (start 126.95 62.04) (end 126.52 61.61) (width 0.5) (layer B.Cu) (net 9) (status 30))
 (segment (start 126.52 60.34) (end 126.6 60.26) (width 0.5) (layer B.Cu) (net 9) (status 30))
 (segment (start 126.52 61.61) (end 126.52 60.34) (width 0.5) (layer B.Cu) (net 9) (status 30))
 (segment (start 127.27 62.04) (end 128.8 60.51) (width 0.5) (layer B.Cu) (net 9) (status 30))
 (segment (start 126.95 62.04) (end 127.27 62.04) (width 0.5) (layer B.Cu) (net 9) (status 30))
 (segment (start 125.7808 63.0492) (end 126.82 62.01) (width 0.5) (layer B.Cu) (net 9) (status 30))
 (segment (start 125.7808 64.0842) (end 125.7808 63.0492) (width 0.5) (layer B.Cu) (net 9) (status 30))
 (segment (start 122.3 60.51) (end 128.8 60.51) (width 0.5) (layer F.Cu) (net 9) (status 30))
 (segment (start 132.679999 65.520001) (end 130.98 67.22) (width 0.5) (layer B.Cu) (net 1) (status 20))
 (segment (start 133.485001 65.520001) (end 132.679999 65.520001) (width 0.5) (layer B.Cu) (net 1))
 (segment (start 135.188 63.817002) (end 133.485001 65.520001) (width 0.5) (layer B.Cu) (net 1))
 (segment (start 135.188 60.69) (end 135.188 63.817002) (width 0.5) (layer B.Cu) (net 1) (status 10))
 (segment (start 130.048 76.832) (end 128.72 78.16) (width 0.5) (layer F.Cu) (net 15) (status 20))
 (segment (start 130.048 75.3488) (end 130.048 76.832) (width 0.5) (layer F.Cu) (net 15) (status 10))
 (segment (start 124.72 57.64) (end 124.7 57.66) (width 0.5) (layer B.Cu) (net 7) (status 30))
 (segment (start 124.72 55.66) (end 124.72 57.64) (width 0.5) (layer B.Cu) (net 7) (status 30))
 (via (at 124.7 57.66) (size 0.8) (drill 0.4) (layers F.Cu B.Cu) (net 7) (status 30))
 (segment (start 122.89844 57.66) (end 124.7 57.66) (width 0.25) (layer F.Cu) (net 7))
 (segment (start 120.69572 59.86272) (end 122.89844 57.66) (width 0.25) (layer F.Cu) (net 7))
 (segment (start 121.998718 62.02172) (end 120.69572 60.718722) (width 0.25) (layer F.Cu) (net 7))
 (segment (start 122.71248 62.02172) (end 121.998718 62.02172) (width 0.25) (layer F.Cu) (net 7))
 (segment (start 124.29236 76.58764) (end 124.29236 72.19696) (width 0.25) (layer F.Cu) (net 7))
 (segment (start 120.69572 60.718722) (end 120.69572 59.86272) (width 0.25) (layer F.Cu) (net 7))
 (segment (start 124.29236 72.19696) (end 126.07544 70.41388) (width 0.25) (layer F.Cu) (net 7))
 (segment (start 126.07544 70.41388) (end 126.07544 67.98564) (width 0.25) (layer F.Cu) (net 7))
 (segment (start 123.73864 65.64884) (end 123.73864 63.64224) (width 0.25) (layer F.Cu) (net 7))
 (segment (start 126.07544 67.98564) (end 123.73864 65.64884) (width 0.25) (layer F.Cu) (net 7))
 (segment (start 124.46 62.92088) (end 125.49124 62.92088) (width 0.25) (layer F.Cu) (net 7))
 (segment (start 123.73864 63.64224) (end 124.46 62.92088) (width 0.25) (layer F.Cu) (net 7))
 (segment (start 122.72 78.16) (end 124.29236 76.58764) (width 0.25) (layer F.Cu) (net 7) (status 10))
 (segment (start 125.68428 62.72784) (end 125.68428 61.449278) (width 0.25) (layer F.Cu) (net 7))
 (segment (start 125.68428 61.449278) (end 125.316922 61.08192) (width 0.25) (layer F.Cu) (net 7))
 (segment (start 125.49124 62.92088) (end 125.68428 62.72784) (width 0.25) (layer F.Cu) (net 7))
 (segment (start 125.316922 61.08192) (end 123.65228 61.08192) (width 0.25) (layer F.Cu) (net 7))
 (segment (start 123.65228 61.08192) (end 122.71248 62.02172) (width 0.25) (layer F.Cu) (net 7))
 (segment (start 123.0376 71.8749) (end 125.0825 69.83) (width 0.5) (layer F.Cu) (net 10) (status 20))
 (segment (start 123.0376 73.0188) (end 123.0376 71.8749) (width 0.5) (layer F.Cu) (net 10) (status 10))
 (segment (start 123.0376 75.8424) (end 120.72 78.16) (width 0.5) (layer F.Cu) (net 13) (status 30))
 (segment (start 123.0376 75.4188) (end 123.0376 75.8424) (width 0.5) (layer F.Cu) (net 13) (status 30))
 (segment (start 131.41 60.495) (end 131.45 60.535) (width 0.5) (layer F.Cu) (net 14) (status 30))
 (segment (start 131.41 58.52) (end 131.41 60.495) (width 0.5) (layer F.Cu) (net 14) (status 30))
 (segment (start 123.13 58.69) (end 124.7 60.26) (width 0.5) (layer B.Cu) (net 8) (status 30))
 (segment (start 122.88 58.69) (end 123.13 58.69) (width 0.5) (layer B.Cu) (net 8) (status 30))
 (segment (start 122.88 56.59) (end 122.3 56.01) (width 0.5) (layer B.Cu) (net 8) (status 30))
 (segment (start 122.88 58.69) (end 122.88 56.59) (width 0.5) (layer B.Cu) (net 8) (status 30))
 (segment (start 128.8 56.01) (end 122.3 56.01) (width 0.5) (layer F.Cu) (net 8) (status 30))
 (segment (start 128.91 56.12) (end 128.8 56.01) (width 0.5) (layer F.Cu) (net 8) (status 30))
 (segment (start 131.41 56.12) (end 128.91 56.12) (width 0.5) (layer F.Cu) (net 8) (status 30))
 (via (at 132.821162 64.111162) (size 0.8) (drill 0.4) (layers F.Cu B.Cu) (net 3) (status 30))
 (segment (start 129.59 66.25) (end 130.682324 66.25) (width 0.5) (layer F.Cu) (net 3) (status 10))
 (segment (start 130.682324 66.25) (end 132.821162 64.111162) (width 0.5) (layer F.Cu) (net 3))
 (segment (start 130.98 61.354) (end 130.98 64.17) (width 0.5) (layer B.Cu) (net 5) (status 30))
 (segment (start 131.484 60.85) (end 130.98 61.354) (width 0.5) (layer B.Cu) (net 5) (status 30))
 (segment (start 128.91 64.53) (end 129.59 63.85) (width 0.5) (layer F.Cu) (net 5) (status 30))
 (segment (start 127.21 64.53) (end 128.91 64.53) (width 0.5) (layer F.Cu) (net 5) (status 30))
 (via (at 130.955824 64.915824) (size 0.8) (drill 0.4) (layers F.Cu B.Cu) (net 5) (status 30))
 (segment (start 129.59 63.85) (end 129.89 63.85) (width 0.5) (layer F.Cu) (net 5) (status 30))
 (segment (start 129.89 63.85) (end 130.955824 64.915824) (width 0.5) (layer F.Cu) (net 5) (status 10))
 (segment (start 128.458011 58.170009) (end 125.774996 58.170009) (width 0.5) (layer F.Cu) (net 6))
 (via (at 125.774996 58.170009) (size 0.8) (drill 0.4) (layers F.Cu B.Cu) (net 6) (status 30))
 (segment (start 125.21 63.58) (end 127.728002 63.58) (width 0.5) (layer F.Cu) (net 6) (status 10))
 (segment (start 127.728002 63.58) (end 130.150001 61.158001) (width 0.5) (layer F.Cu) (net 6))
 (segment (start 130.150001 61.158001) (end 130.150001 59.861999) (width 0.5) (layer F.Cu) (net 6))
 (segment (start 130.150001 59.861999) (end 128.458011 58.170009) (width 0.5) (layer F.Cu) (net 6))
 (segment (start 133.98419 62.23499) (end 135.77828 64.02908) (width 0.5) (layer F.Cu) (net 6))
 (segment (start 131.176444 62.23499) (end 133.98419 62.23499) (width 0.5) (layer F.Cu) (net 6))
 (segment (start 130.150001 61.208547) (end 131.176444 62.23499) (width 0.5) (layer F.Cu) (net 6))
 (segment (start 130.150001 61.158001) (end 130.150001 61.208547) (width 0.5) (layer F.Cu) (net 6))
 (segment (start 134.82828 66.02908) (end 135.423211 66.624011) (width 0.5) (layer F.Cu) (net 12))
 (segment (start 135.423211 66.624011) (end 135.423211 68.056189) (width 0.5) (layer F.Cu) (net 12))
 (segment (start 135.423211 68.056189) (end 134.5438 68.9356) (width 0.5) (layer F.Cu) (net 12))
 (segment (start 135.8265 70.2183) (end 134.5438 68.9356) (width 0.5) (layer F.Cu) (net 12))
 (segment (start 135.8265 79.4385) (end 135.8265 70.2183) (width 0.5) (layer F.Cu) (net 12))
 (segment (start 135.605 79.66) (end 135.8265 79.4385) (width 0.5) (layer F.Cu) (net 12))
 (segment (start 133.32 79.66) (end 135.605 79.66) (width 0.5) (layer F.Cu) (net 12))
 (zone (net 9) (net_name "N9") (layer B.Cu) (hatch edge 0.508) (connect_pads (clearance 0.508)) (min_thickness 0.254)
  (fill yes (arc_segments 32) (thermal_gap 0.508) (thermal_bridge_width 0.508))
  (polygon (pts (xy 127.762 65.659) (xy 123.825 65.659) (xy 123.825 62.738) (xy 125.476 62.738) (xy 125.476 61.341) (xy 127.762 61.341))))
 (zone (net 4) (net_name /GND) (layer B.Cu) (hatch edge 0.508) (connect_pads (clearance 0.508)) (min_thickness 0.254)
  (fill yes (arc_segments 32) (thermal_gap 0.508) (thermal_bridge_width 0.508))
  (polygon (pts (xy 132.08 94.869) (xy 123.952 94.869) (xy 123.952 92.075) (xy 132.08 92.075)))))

